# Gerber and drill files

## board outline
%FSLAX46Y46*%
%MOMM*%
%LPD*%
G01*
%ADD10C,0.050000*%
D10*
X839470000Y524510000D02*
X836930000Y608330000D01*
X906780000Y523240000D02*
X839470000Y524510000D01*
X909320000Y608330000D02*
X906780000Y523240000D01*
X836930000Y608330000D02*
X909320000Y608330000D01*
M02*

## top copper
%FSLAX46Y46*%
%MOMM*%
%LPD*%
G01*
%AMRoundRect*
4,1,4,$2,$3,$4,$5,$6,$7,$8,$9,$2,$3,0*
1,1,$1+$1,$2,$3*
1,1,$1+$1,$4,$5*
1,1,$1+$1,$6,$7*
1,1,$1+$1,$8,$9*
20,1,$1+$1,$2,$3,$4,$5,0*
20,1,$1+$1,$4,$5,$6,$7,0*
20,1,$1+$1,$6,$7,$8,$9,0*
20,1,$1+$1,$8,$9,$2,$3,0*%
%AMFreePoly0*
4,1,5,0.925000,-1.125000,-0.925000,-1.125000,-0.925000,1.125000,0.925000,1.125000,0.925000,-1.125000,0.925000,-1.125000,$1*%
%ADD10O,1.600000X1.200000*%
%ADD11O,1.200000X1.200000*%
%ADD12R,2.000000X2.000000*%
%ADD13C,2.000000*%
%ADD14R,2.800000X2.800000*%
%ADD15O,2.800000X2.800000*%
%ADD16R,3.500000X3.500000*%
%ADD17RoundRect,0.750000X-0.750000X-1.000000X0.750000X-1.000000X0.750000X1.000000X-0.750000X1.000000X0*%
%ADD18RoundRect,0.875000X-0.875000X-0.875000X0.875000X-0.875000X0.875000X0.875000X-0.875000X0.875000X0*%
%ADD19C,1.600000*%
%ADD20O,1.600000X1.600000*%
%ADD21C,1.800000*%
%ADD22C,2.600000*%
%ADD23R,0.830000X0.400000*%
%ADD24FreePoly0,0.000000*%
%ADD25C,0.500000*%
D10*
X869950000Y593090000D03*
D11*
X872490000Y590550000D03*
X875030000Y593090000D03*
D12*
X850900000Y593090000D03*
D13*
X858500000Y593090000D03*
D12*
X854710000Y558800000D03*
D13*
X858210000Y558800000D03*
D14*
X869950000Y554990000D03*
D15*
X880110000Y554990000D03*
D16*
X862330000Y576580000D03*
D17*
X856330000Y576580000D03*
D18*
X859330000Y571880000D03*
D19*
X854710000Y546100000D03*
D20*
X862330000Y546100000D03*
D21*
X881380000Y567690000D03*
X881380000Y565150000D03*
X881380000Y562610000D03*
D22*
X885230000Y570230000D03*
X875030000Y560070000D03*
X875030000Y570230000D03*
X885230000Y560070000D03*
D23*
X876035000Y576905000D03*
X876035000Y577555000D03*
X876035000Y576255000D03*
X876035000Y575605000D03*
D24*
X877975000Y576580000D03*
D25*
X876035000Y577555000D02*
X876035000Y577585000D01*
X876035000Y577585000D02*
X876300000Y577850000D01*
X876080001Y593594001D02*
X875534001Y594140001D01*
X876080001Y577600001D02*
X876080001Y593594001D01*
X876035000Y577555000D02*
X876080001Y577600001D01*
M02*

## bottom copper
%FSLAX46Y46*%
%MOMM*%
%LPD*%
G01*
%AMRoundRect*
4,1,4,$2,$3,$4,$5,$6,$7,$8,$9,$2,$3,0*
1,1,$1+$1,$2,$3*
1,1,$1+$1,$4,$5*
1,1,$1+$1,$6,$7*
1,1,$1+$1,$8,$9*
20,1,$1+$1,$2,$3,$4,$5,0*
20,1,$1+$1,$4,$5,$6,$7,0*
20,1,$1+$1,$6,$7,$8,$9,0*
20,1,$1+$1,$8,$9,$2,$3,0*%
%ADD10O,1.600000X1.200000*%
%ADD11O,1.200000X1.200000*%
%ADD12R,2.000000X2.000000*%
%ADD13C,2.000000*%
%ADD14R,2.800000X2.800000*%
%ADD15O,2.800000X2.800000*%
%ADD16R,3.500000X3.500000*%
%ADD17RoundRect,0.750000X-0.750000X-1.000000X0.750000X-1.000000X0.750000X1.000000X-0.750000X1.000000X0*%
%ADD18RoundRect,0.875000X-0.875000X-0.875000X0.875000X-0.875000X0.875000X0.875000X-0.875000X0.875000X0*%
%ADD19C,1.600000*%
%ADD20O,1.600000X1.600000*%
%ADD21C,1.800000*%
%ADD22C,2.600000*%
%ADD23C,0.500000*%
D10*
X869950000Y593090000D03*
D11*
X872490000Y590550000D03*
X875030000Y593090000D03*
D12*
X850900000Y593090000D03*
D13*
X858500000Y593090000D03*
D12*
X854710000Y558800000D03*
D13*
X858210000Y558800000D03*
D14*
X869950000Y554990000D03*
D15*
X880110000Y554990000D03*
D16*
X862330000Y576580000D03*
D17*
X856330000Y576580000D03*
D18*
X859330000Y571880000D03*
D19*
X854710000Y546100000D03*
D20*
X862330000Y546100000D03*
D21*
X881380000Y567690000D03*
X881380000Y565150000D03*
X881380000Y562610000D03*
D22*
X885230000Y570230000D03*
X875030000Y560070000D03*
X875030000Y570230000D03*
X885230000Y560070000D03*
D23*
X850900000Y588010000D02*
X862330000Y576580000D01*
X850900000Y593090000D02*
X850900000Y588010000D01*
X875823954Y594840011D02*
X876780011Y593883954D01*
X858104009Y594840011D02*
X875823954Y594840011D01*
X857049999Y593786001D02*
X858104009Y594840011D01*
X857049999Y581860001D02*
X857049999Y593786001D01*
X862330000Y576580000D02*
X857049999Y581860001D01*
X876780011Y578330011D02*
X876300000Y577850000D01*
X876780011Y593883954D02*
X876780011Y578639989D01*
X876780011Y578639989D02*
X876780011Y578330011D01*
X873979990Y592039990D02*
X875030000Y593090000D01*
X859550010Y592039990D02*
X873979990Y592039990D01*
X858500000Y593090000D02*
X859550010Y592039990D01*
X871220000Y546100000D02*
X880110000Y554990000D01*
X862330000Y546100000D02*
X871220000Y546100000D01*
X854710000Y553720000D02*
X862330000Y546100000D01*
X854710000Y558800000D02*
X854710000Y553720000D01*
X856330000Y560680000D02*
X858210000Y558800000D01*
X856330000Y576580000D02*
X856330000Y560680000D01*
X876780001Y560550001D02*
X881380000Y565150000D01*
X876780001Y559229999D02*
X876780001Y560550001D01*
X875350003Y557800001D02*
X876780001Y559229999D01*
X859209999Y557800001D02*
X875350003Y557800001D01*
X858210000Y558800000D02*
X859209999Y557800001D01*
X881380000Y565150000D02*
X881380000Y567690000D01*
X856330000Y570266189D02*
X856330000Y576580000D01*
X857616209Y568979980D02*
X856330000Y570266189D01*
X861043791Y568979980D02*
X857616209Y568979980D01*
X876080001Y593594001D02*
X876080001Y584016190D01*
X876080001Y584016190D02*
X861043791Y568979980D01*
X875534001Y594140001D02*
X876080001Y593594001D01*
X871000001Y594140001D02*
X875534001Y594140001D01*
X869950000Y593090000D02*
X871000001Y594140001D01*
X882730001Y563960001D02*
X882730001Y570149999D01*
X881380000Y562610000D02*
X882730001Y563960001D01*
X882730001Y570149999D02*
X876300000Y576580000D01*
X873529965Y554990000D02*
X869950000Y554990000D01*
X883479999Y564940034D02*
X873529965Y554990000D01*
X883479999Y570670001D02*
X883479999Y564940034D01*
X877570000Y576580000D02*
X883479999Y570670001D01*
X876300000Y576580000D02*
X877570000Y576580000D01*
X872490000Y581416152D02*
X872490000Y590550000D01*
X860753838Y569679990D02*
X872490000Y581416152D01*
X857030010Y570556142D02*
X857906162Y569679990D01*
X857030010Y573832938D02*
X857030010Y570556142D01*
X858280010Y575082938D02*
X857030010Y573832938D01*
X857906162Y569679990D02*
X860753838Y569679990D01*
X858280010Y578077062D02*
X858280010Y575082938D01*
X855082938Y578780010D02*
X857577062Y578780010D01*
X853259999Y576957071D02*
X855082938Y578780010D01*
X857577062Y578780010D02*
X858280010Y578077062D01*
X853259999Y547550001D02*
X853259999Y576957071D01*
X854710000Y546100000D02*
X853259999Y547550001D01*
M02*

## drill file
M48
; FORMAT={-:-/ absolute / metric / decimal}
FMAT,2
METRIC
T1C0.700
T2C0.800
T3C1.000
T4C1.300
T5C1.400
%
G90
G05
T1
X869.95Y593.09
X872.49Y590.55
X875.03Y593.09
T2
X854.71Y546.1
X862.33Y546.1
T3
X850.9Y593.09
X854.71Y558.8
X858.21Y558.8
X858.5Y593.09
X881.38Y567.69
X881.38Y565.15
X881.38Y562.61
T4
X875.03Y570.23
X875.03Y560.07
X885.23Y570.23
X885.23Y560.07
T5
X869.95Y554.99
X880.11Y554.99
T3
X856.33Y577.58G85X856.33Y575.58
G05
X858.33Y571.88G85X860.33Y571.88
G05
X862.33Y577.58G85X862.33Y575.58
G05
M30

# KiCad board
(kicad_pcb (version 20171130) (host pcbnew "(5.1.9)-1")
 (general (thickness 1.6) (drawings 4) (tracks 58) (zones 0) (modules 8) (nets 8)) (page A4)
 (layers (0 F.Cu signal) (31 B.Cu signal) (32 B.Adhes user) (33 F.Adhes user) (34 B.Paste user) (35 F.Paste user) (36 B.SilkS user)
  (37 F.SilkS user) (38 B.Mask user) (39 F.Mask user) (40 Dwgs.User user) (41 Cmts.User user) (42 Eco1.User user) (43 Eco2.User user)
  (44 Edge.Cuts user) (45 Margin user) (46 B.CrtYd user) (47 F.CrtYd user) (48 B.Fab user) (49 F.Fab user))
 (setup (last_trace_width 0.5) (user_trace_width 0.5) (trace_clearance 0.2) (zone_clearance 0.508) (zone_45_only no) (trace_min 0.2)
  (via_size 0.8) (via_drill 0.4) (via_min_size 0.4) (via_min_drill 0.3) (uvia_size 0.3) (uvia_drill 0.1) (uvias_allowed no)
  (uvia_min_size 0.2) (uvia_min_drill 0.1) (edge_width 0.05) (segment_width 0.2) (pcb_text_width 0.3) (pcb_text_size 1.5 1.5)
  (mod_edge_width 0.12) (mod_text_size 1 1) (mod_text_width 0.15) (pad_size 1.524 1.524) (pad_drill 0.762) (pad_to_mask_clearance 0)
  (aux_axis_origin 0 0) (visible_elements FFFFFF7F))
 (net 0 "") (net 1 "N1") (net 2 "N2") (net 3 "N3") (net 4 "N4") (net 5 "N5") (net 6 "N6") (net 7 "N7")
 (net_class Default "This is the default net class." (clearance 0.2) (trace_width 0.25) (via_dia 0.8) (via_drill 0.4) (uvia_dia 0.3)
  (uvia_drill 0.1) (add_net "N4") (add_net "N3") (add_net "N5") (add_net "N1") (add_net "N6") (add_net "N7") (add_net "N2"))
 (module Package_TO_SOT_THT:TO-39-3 (layer F.Cu) (at 869.95 -593.09)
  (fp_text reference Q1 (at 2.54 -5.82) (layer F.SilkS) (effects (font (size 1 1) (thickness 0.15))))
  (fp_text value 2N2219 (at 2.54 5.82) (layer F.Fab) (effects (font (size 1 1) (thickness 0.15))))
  (pad 1 thru_hole oval (at 0 0) (size 1.6 1.2) (drill 0.7) (layers *.Cu *.Mask) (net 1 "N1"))
  (pad 2 thru_hole oval (at 2.54 2.54) (size 1.2 1.2) (drill 0.7) (layers *.Cu *.Mask) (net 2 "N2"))
  (pad 3 thru_hole oval (at 5.08 0) (size 1.2 1.2) (drill 0.7) (layers *.Cu *.Mask) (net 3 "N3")))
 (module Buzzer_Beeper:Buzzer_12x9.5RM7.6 (layer F.Cu) (at 850.9 -593.09)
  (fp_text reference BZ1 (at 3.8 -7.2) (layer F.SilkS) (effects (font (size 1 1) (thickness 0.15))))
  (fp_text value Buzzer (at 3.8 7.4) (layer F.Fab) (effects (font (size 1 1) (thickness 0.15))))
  (pad 1 thru_hole rect (at 0 0) (size 2 2) (drill 1) (layers *.Cu *.Mask) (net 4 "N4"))
  (pad 2 thru_hole circle (at 7.6 0) (size 2 2) (drill 1) (layers *.Cu *.Mask) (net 3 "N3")))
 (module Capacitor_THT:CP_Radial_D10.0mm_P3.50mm (layer F.Cu) (at 854.71 -558.8)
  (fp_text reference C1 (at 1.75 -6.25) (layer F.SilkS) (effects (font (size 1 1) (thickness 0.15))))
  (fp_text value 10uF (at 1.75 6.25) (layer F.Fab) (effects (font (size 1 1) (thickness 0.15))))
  (pad 1 thru_hole rect (at 0 0) (size 2 2) (drill 1) (layers *.Cu *.Mask) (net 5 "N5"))
  (pad 2 thru_hole circle (at 3.5 0) (size 2 2) (drill 1) (layers *.Cu *.Mask) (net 1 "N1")))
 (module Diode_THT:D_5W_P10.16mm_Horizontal (layer F.Cu) (at 869.95 -554.99)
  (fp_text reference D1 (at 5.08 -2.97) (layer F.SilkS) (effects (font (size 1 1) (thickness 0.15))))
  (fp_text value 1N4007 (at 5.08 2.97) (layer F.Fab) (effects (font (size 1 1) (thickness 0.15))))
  (pad 1 thru_hole rect (at 0 0) (size 2.8 2.8) (drill 1.4) (layers *.Cu *.Mask) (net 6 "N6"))
  (pad 2 thru_hole oval (at 10.16 0) (size 2.8 2.8) (drill 1.4) (layers *.Cu *.Mask) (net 5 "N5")))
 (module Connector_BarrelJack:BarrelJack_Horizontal (layer F.Cu) (at 862.33 -576.58)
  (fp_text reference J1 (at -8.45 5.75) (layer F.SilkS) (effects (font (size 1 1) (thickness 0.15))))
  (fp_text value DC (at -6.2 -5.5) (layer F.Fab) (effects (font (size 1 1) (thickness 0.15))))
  (pad 1 thru_hole rect (at 0 0) (size 3.5 3.5) (drill oval 1 3) (layers *.Cu *.Mask) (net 4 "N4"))
  (pad 2 thru_hole roundrect (at -6 0) (size 3 3.5) (drill oval 1 3) (layers *.Cu *.Mask) (roundrect_rratio 0.25) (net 1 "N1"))
  (pad 3 thru_hole roundrect (at -3 4.7) (size 3.5 3.5) (drill oval 3 1) (layers *.Cu *.Mask) (roundrect_rratio 0.25) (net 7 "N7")))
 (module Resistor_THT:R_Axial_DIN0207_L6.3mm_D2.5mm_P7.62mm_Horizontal (layer F.Cu) (at 854.71 -546.1)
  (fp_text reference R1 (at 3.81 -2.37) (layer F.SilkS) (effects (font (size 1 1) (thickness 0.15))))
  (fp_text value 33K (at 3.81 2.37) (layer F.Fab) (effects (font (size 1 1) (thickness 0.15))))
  (pad 1 thru_hole circle (at 0 0) (size 1.6 1.6) (drill 0.8) (layers *.Cu *.Mask) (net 2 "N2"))
  (pad 2 thru_hole oval (at 7.62 0) (size 1.6 1.6) (drill 0.8) (layers *.Cu *.Mask) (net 5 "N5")))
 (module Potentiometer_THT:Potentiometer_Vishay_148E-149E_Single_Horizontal (layer F.Cu) (at 881.38 -562.61)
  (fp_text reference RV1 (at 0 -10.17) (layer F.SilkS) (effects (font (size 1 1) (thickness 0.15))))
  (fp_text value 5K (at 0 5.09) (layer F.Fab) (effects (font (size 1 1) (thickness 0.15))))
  (pad 3 thru_hole circle (at 0 -5.08) (size 1.8 1.8) (drill 1) (layers *.Cu *.Mask) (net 1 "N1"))
  (pad 2 thru_hole circle (at 0 -2.54) (size 1.8 1.8) (drill 1) (layers *.Cu *.Mask) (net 1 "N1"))
  (pad 1 thru_hole circle (at 0 0) (size 1.8 1.8) (drill 1) (layers *.Cu *.Mask) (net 6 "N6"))
  (pad "" thru_hole circle (at 3.85 -7.62) (size 2.6 2.6) (drill 1.3) (layers *.Cu *.Mask))
  (pad "" thru_hole circle (at -6.35 2.54) (size 2.6 2.6) (drill 1.3) (layers *.Cu *.Mask))
  (pad "" thru_hole circle (at -6.35 -7.62) (size 2.6 2.6) (drill 1.3) (layers *.Cu *.Mask))
  (pad "" thru_hole circle (at 3.85 2.54) (size 2.6 2.6) (drill 1.3) (layers *.Cu *.Mask)))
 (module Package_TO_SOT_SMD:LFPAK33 (layer F.Cu) (at 877.57 -576.58) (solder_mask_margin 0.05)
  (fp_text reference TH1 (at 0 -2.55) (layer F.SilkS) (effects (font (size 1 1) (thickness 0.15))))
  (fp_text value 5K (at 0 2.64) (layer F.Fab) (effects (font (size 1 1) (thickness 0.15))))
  (pad "" smd rect (at -0.215 -0.626) (size 0.51 0.635) (layers F.Paste))
  (pad "" smd rect (at 0.645 -0.626) (size 0.51 0.635) (layers F.Paste))
  (pad "" smd rect (at -0.215 0.626) (size 0.51 0.635) (layers F.Paste))
  (pad "" smd rect (at 0.645 0.626) (size 0.51 0.635) (layers F.Paste))
  (pad 2 smd rect (at -1.535 -0.325) (size 0.83 0.4) (layers F.Cu F.Mask) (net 6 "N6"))
  (pad 1 smd rect (at -1.535 -0.975) (size 0.83 0.4) (layers F.Cu F.Mask) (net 4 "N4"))
  (pad 3 smd rect (at -1.535 0.325) (size 0.83 0.4) (layers F.Cu F.Mask))
  (pad "" smd rect (at -1.535 0.975) (size 0.83 0.3) (layers F.Paste))
  (pad 4 smd rect (at -1.535 0.975) (size 0.83 0.4) (layers F.Cu F.Mask))
  (pad "" smd rect (at -1.535 0.325) (size 0.83 0.3) (layers F.Paste))
  (pad "" smd rect (at -1.535 -0.325) (size 0.83 0.3) (layers F.Paste))
  (pad "" smd rect (at -1.535 -0.975) (size 0.83 0.3) (layers F.Paste))
  (pad "" smd rect (at 1.575 -0.975) (size 0.75 0.3) (layers F.Paste))
  (pad "" smd rect (at 1.575 -0.325) (size 0.75 0.3) (layers F.Paste))
  (pad "" smd rect (at 1.575 0.325) (size 0.75 0.3) (layers F.Paste))
  (pad "" smd rect (at 1.575 0.975) (size 0.75 0.3) (layers F.Paste))
  (pad 5 smd custom (at 0.405 0) (size 1.85 2.25) (layers F.Cu F.Mask) (zone_connect 2) (options (clearance outline) (anchor rect))
   (primitives)))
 (gr_line (start 839.47 -524.51) (end 836.93 -608.33) (layer Edge.Cuts) (width 0.05))
 (gr_line (start 906.78 -523.24) (end 839.47 -524.51) (layer Edge.Cuts) (width 0.05))
 (gr_line (start 909.32 -608.33) (end 906.78 -523.24) (layer Edge.Cuts) (width 0.05))
 (gr_line (start 836.93 -608.33) (end 909.32 -608.33) (layer Edge.Cuts) (width 0.05))
 (segment (start 850.9 -588.01) (end 862.33 -576.58) (width 0.5) (layer B.Cu) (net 4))
 (segment (start 850.9 -593.09) (end 850.9 -588.01) (width 0.5) (layer B.Cu) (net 4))
 (segment (start 875.823954 -594.840011) (end 876.780011 -593.883954) (width 0.5) (layer B.Cu) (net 4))
 (segment (start 858.104009 -594.840011) (end 875.823954 -594.840011) (width 0.5) (layer B.Cu) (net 4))
 (segment (start 857.049999 -593.786001) (end 858.104009 -594.840011) (width 0.5) (layer B.Cu) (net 4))
 (segment (start 857.049999 -581.860001) (end 857.049999 -593.786001) (width 0.5) (layer B.Cu) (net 4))
 (segment (start 862.33 -576.58) (end 857.049999 -581.860001) (width 0.5) (layer B.Cu) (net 4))
 (segment (start 876.780011 -578.330011) (end 876.3 -577.85) (width 0.5) (layer B.Cu) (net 4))
 (segment (start 876.035 -577.555) (end 876.035 -577.585) (width 0.5) (layer F.Cu) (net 4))
 (segment (start 876.035 -577.585) (end 876.3 -577.85) (width 0.5) (layer F.Cu) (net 4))
 (segment (start 876.080001 -593.594001) (end 875.534001 -594.140001) (width 0.5) (layer F.Cu) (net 4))
 (segment (start 876.080001 -577.600001) (end 876.080001 -593.594001) (width 0.5) (layer F.Cu) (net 4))
 (segment (start 876.035 -577.555) (end 876.080001 -577.600001) (width 0.5) (layer F.Cu) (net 4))
 (segment (start 876.780011 -593.883954) (end 876.780011 -578.639989) (width 0.5) (layer B.Cu) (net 4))
 (segment (start 876.780011 -578.639989) (end 876.780011 -578.330011) (width 0.5) (layer B.Cu) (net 4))
 (segment (start 873.97999 -592.03999) (end 875.03 -593.09) (width 0.5) (layer B.Cu) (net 3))
 (segment (start 859.55001 -592.03999) (end 873.97999 -592.03999) (width 0.5) (layer B.Cu) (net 3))
 (segment (start 858.5 -593.09) (end 859.55001 -592.03999) (width 0.5) (layer B.Cu) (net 3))
 (segment (start 871.22 -546.1) (end 880.11 -554.99) (width 0.5) (layer B.Cu) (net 5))
 (segment (start 862.33 -546.1) (end 871.22 -546.1) (width 0.5) (layer B.Cu) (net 5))
 (segment (start 854.71 -553.72) (end 862.33 -546.1) (width 0.5) (layer B.Cu) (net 5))
 (segment (start 854.71 -558.8) (end 854.71 -553.72) (width 0.5) (layer B.Cu) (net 5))
 (segment (start 856.33 -560.68) (end 858.21 -558.8) (width 0.5) (layer B.Cu) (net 1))
 (segment (start 856.33 -576.58) (end 856.33 -560.68) (width 0.5) (layer B.Cu) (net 1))
 (segment (start 876.780001 -560.550001) (end 881.38 -565.15) (width 0.5) (layer B.Cu) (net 1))
 (segment (start 876.780001 -559.229999) (end 876.780001 -560.550001) (width 0.5) (layer B.Cu) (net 1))
 (segment (start 875.350003 -557.800001) (end 876.780001 -559.229999) (width 0.5) (layer B.Cu) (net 1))
 (segment (start 859.209999 -557.800001) (end 875.350003 -557.800001) (width 0.5) (layer B.Cu) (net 1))
 (segment (start 858.21 -558.8) (end 859.209999 -557.800001) (width 0.5) (layer B.Cu) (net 1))
 (segment (start 881.38 -565.15) (end 881.38 -567.69) (width 0.5) (layer B.Cu) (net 1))
 (segment (start 856.33 -570.266189) (end 856.33 -576.58) (width 0.5) (layer B.Cu) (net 1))
 (segment (start 857.616209 -568.97998) (end 856.33 -570.266189) (width 0.5) (layer B.Cu) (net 1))
 (segment (start 861.043791 -568.97998) (end 857.616209 -568.97998) (width 0.5) (layer B.Cu) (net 1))
 (segment (start 876.080001 -593.594001) (end 876.080001 -584.01619) (width 0.5) (layer B.Cu) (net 1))
 (segment (start 876.080001 -584.01619) (end 861.043791 -568.97998) (width 0.5) (layer B.Cu) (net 1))
 (segment (start 875.534001 -594.140001) (end 876.080001 -593.594001) (width 0.5) (layer B.Cu) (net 1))
 (segment (start 871.000001 -594.140001) (end 875.534001 -594.140001) (width 0.5) (layer B.Cu) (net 1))
 (segment (start 869.95 -593.09) (end 871.000001 -594.140001) (width 0.5) (layer B.Cu) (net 1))
 (segment (start 882.730001 -563.960001) (end 882.730001 -570.149999) (width 0.5) (layer B.Cu) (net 6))
 (segment (start 881.38 -562.61) (end 882.730001 -563.960001) (width 0.5) (layer B.Cu) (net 6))
 (segment (start 882.730001 -570.149999) (end 876.3 -576.58) (width 0.5) (layer B.Cu) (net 6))
 (segment (start 873.529965 -554.99) (end 869.95 -554.99) (width 0.5) (layer B.Cu) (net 6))
 (segment (start 883.479999 -564.940034) (end 873.529965 -554.99) (width 0.5) (layer B.Cu) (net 6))
 (segment (start 883.479999 -570.670001) (end 883.479999 -564.940034) (width 0.5) (layer B.Cu) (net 6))
 (segment (start 877.57 -576.58) (end 883.479999 -570.670001) (width 0.5) (layer B.Cu) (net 6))
 (segment (start 876.3 -576.58) (end 877.57 -576.58) (width 0.5) (layer B.Cu) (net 6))
 (segment (start 872.49 -581.416152) (end 872.49 -590.55) (width 0.5) (layer B.Cu) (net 2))
 (segment (start 860.753838 -569.67999) (end 872.49 -581.416152) (width 0.5) (layer B.Cu) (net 2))
 (segment (start 857.03001 -570.556142) (end 857.906162 -569.67999) (width 0.5) (layer B.Cu) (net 2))
 (segment (start 857.03001 -573.832938) (end 857.03001 -570.556142) (width 0.5) (layer B.Cu) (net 2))
 (segment (start 858.28001 -575.082938) (end 857.03001 -573.832938) (width 0.5) (layer B.Cu) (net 2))
 (segment (start 857.906162 -569.67999) (end 860.753838 -569.67999) (width 0.5) (layer B.Cu) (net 2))
 (segment (start 858.28001 -578.077062) (end 858.28001 -575.082938) (width 0.5) (layer B.Cu) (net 2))
 (segment (start 855.082938 -578.78001) (end 857.577062 -578.78001) (width 0.5) (layer B.Cu) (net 2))
 (segment (start 853.259999 -576.957071) (end 855.082938 -578.78001) (width 0.5) (layer B.Cu) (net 2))
 (segment (start 857.577062 -578.78001) (end 858.28001 -578.077062) (width 0.5) (layer B.Cu) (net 2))
 (segment (start 853.259999 -547.550001) (end 853.259999 -576.957071) (width 0.5) (layer B.Cu) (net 2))
 (segment (start 854.71 -546.1) (end 853.259999 -547.550001) (width 0.5) (layer B.Cu) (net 2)))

